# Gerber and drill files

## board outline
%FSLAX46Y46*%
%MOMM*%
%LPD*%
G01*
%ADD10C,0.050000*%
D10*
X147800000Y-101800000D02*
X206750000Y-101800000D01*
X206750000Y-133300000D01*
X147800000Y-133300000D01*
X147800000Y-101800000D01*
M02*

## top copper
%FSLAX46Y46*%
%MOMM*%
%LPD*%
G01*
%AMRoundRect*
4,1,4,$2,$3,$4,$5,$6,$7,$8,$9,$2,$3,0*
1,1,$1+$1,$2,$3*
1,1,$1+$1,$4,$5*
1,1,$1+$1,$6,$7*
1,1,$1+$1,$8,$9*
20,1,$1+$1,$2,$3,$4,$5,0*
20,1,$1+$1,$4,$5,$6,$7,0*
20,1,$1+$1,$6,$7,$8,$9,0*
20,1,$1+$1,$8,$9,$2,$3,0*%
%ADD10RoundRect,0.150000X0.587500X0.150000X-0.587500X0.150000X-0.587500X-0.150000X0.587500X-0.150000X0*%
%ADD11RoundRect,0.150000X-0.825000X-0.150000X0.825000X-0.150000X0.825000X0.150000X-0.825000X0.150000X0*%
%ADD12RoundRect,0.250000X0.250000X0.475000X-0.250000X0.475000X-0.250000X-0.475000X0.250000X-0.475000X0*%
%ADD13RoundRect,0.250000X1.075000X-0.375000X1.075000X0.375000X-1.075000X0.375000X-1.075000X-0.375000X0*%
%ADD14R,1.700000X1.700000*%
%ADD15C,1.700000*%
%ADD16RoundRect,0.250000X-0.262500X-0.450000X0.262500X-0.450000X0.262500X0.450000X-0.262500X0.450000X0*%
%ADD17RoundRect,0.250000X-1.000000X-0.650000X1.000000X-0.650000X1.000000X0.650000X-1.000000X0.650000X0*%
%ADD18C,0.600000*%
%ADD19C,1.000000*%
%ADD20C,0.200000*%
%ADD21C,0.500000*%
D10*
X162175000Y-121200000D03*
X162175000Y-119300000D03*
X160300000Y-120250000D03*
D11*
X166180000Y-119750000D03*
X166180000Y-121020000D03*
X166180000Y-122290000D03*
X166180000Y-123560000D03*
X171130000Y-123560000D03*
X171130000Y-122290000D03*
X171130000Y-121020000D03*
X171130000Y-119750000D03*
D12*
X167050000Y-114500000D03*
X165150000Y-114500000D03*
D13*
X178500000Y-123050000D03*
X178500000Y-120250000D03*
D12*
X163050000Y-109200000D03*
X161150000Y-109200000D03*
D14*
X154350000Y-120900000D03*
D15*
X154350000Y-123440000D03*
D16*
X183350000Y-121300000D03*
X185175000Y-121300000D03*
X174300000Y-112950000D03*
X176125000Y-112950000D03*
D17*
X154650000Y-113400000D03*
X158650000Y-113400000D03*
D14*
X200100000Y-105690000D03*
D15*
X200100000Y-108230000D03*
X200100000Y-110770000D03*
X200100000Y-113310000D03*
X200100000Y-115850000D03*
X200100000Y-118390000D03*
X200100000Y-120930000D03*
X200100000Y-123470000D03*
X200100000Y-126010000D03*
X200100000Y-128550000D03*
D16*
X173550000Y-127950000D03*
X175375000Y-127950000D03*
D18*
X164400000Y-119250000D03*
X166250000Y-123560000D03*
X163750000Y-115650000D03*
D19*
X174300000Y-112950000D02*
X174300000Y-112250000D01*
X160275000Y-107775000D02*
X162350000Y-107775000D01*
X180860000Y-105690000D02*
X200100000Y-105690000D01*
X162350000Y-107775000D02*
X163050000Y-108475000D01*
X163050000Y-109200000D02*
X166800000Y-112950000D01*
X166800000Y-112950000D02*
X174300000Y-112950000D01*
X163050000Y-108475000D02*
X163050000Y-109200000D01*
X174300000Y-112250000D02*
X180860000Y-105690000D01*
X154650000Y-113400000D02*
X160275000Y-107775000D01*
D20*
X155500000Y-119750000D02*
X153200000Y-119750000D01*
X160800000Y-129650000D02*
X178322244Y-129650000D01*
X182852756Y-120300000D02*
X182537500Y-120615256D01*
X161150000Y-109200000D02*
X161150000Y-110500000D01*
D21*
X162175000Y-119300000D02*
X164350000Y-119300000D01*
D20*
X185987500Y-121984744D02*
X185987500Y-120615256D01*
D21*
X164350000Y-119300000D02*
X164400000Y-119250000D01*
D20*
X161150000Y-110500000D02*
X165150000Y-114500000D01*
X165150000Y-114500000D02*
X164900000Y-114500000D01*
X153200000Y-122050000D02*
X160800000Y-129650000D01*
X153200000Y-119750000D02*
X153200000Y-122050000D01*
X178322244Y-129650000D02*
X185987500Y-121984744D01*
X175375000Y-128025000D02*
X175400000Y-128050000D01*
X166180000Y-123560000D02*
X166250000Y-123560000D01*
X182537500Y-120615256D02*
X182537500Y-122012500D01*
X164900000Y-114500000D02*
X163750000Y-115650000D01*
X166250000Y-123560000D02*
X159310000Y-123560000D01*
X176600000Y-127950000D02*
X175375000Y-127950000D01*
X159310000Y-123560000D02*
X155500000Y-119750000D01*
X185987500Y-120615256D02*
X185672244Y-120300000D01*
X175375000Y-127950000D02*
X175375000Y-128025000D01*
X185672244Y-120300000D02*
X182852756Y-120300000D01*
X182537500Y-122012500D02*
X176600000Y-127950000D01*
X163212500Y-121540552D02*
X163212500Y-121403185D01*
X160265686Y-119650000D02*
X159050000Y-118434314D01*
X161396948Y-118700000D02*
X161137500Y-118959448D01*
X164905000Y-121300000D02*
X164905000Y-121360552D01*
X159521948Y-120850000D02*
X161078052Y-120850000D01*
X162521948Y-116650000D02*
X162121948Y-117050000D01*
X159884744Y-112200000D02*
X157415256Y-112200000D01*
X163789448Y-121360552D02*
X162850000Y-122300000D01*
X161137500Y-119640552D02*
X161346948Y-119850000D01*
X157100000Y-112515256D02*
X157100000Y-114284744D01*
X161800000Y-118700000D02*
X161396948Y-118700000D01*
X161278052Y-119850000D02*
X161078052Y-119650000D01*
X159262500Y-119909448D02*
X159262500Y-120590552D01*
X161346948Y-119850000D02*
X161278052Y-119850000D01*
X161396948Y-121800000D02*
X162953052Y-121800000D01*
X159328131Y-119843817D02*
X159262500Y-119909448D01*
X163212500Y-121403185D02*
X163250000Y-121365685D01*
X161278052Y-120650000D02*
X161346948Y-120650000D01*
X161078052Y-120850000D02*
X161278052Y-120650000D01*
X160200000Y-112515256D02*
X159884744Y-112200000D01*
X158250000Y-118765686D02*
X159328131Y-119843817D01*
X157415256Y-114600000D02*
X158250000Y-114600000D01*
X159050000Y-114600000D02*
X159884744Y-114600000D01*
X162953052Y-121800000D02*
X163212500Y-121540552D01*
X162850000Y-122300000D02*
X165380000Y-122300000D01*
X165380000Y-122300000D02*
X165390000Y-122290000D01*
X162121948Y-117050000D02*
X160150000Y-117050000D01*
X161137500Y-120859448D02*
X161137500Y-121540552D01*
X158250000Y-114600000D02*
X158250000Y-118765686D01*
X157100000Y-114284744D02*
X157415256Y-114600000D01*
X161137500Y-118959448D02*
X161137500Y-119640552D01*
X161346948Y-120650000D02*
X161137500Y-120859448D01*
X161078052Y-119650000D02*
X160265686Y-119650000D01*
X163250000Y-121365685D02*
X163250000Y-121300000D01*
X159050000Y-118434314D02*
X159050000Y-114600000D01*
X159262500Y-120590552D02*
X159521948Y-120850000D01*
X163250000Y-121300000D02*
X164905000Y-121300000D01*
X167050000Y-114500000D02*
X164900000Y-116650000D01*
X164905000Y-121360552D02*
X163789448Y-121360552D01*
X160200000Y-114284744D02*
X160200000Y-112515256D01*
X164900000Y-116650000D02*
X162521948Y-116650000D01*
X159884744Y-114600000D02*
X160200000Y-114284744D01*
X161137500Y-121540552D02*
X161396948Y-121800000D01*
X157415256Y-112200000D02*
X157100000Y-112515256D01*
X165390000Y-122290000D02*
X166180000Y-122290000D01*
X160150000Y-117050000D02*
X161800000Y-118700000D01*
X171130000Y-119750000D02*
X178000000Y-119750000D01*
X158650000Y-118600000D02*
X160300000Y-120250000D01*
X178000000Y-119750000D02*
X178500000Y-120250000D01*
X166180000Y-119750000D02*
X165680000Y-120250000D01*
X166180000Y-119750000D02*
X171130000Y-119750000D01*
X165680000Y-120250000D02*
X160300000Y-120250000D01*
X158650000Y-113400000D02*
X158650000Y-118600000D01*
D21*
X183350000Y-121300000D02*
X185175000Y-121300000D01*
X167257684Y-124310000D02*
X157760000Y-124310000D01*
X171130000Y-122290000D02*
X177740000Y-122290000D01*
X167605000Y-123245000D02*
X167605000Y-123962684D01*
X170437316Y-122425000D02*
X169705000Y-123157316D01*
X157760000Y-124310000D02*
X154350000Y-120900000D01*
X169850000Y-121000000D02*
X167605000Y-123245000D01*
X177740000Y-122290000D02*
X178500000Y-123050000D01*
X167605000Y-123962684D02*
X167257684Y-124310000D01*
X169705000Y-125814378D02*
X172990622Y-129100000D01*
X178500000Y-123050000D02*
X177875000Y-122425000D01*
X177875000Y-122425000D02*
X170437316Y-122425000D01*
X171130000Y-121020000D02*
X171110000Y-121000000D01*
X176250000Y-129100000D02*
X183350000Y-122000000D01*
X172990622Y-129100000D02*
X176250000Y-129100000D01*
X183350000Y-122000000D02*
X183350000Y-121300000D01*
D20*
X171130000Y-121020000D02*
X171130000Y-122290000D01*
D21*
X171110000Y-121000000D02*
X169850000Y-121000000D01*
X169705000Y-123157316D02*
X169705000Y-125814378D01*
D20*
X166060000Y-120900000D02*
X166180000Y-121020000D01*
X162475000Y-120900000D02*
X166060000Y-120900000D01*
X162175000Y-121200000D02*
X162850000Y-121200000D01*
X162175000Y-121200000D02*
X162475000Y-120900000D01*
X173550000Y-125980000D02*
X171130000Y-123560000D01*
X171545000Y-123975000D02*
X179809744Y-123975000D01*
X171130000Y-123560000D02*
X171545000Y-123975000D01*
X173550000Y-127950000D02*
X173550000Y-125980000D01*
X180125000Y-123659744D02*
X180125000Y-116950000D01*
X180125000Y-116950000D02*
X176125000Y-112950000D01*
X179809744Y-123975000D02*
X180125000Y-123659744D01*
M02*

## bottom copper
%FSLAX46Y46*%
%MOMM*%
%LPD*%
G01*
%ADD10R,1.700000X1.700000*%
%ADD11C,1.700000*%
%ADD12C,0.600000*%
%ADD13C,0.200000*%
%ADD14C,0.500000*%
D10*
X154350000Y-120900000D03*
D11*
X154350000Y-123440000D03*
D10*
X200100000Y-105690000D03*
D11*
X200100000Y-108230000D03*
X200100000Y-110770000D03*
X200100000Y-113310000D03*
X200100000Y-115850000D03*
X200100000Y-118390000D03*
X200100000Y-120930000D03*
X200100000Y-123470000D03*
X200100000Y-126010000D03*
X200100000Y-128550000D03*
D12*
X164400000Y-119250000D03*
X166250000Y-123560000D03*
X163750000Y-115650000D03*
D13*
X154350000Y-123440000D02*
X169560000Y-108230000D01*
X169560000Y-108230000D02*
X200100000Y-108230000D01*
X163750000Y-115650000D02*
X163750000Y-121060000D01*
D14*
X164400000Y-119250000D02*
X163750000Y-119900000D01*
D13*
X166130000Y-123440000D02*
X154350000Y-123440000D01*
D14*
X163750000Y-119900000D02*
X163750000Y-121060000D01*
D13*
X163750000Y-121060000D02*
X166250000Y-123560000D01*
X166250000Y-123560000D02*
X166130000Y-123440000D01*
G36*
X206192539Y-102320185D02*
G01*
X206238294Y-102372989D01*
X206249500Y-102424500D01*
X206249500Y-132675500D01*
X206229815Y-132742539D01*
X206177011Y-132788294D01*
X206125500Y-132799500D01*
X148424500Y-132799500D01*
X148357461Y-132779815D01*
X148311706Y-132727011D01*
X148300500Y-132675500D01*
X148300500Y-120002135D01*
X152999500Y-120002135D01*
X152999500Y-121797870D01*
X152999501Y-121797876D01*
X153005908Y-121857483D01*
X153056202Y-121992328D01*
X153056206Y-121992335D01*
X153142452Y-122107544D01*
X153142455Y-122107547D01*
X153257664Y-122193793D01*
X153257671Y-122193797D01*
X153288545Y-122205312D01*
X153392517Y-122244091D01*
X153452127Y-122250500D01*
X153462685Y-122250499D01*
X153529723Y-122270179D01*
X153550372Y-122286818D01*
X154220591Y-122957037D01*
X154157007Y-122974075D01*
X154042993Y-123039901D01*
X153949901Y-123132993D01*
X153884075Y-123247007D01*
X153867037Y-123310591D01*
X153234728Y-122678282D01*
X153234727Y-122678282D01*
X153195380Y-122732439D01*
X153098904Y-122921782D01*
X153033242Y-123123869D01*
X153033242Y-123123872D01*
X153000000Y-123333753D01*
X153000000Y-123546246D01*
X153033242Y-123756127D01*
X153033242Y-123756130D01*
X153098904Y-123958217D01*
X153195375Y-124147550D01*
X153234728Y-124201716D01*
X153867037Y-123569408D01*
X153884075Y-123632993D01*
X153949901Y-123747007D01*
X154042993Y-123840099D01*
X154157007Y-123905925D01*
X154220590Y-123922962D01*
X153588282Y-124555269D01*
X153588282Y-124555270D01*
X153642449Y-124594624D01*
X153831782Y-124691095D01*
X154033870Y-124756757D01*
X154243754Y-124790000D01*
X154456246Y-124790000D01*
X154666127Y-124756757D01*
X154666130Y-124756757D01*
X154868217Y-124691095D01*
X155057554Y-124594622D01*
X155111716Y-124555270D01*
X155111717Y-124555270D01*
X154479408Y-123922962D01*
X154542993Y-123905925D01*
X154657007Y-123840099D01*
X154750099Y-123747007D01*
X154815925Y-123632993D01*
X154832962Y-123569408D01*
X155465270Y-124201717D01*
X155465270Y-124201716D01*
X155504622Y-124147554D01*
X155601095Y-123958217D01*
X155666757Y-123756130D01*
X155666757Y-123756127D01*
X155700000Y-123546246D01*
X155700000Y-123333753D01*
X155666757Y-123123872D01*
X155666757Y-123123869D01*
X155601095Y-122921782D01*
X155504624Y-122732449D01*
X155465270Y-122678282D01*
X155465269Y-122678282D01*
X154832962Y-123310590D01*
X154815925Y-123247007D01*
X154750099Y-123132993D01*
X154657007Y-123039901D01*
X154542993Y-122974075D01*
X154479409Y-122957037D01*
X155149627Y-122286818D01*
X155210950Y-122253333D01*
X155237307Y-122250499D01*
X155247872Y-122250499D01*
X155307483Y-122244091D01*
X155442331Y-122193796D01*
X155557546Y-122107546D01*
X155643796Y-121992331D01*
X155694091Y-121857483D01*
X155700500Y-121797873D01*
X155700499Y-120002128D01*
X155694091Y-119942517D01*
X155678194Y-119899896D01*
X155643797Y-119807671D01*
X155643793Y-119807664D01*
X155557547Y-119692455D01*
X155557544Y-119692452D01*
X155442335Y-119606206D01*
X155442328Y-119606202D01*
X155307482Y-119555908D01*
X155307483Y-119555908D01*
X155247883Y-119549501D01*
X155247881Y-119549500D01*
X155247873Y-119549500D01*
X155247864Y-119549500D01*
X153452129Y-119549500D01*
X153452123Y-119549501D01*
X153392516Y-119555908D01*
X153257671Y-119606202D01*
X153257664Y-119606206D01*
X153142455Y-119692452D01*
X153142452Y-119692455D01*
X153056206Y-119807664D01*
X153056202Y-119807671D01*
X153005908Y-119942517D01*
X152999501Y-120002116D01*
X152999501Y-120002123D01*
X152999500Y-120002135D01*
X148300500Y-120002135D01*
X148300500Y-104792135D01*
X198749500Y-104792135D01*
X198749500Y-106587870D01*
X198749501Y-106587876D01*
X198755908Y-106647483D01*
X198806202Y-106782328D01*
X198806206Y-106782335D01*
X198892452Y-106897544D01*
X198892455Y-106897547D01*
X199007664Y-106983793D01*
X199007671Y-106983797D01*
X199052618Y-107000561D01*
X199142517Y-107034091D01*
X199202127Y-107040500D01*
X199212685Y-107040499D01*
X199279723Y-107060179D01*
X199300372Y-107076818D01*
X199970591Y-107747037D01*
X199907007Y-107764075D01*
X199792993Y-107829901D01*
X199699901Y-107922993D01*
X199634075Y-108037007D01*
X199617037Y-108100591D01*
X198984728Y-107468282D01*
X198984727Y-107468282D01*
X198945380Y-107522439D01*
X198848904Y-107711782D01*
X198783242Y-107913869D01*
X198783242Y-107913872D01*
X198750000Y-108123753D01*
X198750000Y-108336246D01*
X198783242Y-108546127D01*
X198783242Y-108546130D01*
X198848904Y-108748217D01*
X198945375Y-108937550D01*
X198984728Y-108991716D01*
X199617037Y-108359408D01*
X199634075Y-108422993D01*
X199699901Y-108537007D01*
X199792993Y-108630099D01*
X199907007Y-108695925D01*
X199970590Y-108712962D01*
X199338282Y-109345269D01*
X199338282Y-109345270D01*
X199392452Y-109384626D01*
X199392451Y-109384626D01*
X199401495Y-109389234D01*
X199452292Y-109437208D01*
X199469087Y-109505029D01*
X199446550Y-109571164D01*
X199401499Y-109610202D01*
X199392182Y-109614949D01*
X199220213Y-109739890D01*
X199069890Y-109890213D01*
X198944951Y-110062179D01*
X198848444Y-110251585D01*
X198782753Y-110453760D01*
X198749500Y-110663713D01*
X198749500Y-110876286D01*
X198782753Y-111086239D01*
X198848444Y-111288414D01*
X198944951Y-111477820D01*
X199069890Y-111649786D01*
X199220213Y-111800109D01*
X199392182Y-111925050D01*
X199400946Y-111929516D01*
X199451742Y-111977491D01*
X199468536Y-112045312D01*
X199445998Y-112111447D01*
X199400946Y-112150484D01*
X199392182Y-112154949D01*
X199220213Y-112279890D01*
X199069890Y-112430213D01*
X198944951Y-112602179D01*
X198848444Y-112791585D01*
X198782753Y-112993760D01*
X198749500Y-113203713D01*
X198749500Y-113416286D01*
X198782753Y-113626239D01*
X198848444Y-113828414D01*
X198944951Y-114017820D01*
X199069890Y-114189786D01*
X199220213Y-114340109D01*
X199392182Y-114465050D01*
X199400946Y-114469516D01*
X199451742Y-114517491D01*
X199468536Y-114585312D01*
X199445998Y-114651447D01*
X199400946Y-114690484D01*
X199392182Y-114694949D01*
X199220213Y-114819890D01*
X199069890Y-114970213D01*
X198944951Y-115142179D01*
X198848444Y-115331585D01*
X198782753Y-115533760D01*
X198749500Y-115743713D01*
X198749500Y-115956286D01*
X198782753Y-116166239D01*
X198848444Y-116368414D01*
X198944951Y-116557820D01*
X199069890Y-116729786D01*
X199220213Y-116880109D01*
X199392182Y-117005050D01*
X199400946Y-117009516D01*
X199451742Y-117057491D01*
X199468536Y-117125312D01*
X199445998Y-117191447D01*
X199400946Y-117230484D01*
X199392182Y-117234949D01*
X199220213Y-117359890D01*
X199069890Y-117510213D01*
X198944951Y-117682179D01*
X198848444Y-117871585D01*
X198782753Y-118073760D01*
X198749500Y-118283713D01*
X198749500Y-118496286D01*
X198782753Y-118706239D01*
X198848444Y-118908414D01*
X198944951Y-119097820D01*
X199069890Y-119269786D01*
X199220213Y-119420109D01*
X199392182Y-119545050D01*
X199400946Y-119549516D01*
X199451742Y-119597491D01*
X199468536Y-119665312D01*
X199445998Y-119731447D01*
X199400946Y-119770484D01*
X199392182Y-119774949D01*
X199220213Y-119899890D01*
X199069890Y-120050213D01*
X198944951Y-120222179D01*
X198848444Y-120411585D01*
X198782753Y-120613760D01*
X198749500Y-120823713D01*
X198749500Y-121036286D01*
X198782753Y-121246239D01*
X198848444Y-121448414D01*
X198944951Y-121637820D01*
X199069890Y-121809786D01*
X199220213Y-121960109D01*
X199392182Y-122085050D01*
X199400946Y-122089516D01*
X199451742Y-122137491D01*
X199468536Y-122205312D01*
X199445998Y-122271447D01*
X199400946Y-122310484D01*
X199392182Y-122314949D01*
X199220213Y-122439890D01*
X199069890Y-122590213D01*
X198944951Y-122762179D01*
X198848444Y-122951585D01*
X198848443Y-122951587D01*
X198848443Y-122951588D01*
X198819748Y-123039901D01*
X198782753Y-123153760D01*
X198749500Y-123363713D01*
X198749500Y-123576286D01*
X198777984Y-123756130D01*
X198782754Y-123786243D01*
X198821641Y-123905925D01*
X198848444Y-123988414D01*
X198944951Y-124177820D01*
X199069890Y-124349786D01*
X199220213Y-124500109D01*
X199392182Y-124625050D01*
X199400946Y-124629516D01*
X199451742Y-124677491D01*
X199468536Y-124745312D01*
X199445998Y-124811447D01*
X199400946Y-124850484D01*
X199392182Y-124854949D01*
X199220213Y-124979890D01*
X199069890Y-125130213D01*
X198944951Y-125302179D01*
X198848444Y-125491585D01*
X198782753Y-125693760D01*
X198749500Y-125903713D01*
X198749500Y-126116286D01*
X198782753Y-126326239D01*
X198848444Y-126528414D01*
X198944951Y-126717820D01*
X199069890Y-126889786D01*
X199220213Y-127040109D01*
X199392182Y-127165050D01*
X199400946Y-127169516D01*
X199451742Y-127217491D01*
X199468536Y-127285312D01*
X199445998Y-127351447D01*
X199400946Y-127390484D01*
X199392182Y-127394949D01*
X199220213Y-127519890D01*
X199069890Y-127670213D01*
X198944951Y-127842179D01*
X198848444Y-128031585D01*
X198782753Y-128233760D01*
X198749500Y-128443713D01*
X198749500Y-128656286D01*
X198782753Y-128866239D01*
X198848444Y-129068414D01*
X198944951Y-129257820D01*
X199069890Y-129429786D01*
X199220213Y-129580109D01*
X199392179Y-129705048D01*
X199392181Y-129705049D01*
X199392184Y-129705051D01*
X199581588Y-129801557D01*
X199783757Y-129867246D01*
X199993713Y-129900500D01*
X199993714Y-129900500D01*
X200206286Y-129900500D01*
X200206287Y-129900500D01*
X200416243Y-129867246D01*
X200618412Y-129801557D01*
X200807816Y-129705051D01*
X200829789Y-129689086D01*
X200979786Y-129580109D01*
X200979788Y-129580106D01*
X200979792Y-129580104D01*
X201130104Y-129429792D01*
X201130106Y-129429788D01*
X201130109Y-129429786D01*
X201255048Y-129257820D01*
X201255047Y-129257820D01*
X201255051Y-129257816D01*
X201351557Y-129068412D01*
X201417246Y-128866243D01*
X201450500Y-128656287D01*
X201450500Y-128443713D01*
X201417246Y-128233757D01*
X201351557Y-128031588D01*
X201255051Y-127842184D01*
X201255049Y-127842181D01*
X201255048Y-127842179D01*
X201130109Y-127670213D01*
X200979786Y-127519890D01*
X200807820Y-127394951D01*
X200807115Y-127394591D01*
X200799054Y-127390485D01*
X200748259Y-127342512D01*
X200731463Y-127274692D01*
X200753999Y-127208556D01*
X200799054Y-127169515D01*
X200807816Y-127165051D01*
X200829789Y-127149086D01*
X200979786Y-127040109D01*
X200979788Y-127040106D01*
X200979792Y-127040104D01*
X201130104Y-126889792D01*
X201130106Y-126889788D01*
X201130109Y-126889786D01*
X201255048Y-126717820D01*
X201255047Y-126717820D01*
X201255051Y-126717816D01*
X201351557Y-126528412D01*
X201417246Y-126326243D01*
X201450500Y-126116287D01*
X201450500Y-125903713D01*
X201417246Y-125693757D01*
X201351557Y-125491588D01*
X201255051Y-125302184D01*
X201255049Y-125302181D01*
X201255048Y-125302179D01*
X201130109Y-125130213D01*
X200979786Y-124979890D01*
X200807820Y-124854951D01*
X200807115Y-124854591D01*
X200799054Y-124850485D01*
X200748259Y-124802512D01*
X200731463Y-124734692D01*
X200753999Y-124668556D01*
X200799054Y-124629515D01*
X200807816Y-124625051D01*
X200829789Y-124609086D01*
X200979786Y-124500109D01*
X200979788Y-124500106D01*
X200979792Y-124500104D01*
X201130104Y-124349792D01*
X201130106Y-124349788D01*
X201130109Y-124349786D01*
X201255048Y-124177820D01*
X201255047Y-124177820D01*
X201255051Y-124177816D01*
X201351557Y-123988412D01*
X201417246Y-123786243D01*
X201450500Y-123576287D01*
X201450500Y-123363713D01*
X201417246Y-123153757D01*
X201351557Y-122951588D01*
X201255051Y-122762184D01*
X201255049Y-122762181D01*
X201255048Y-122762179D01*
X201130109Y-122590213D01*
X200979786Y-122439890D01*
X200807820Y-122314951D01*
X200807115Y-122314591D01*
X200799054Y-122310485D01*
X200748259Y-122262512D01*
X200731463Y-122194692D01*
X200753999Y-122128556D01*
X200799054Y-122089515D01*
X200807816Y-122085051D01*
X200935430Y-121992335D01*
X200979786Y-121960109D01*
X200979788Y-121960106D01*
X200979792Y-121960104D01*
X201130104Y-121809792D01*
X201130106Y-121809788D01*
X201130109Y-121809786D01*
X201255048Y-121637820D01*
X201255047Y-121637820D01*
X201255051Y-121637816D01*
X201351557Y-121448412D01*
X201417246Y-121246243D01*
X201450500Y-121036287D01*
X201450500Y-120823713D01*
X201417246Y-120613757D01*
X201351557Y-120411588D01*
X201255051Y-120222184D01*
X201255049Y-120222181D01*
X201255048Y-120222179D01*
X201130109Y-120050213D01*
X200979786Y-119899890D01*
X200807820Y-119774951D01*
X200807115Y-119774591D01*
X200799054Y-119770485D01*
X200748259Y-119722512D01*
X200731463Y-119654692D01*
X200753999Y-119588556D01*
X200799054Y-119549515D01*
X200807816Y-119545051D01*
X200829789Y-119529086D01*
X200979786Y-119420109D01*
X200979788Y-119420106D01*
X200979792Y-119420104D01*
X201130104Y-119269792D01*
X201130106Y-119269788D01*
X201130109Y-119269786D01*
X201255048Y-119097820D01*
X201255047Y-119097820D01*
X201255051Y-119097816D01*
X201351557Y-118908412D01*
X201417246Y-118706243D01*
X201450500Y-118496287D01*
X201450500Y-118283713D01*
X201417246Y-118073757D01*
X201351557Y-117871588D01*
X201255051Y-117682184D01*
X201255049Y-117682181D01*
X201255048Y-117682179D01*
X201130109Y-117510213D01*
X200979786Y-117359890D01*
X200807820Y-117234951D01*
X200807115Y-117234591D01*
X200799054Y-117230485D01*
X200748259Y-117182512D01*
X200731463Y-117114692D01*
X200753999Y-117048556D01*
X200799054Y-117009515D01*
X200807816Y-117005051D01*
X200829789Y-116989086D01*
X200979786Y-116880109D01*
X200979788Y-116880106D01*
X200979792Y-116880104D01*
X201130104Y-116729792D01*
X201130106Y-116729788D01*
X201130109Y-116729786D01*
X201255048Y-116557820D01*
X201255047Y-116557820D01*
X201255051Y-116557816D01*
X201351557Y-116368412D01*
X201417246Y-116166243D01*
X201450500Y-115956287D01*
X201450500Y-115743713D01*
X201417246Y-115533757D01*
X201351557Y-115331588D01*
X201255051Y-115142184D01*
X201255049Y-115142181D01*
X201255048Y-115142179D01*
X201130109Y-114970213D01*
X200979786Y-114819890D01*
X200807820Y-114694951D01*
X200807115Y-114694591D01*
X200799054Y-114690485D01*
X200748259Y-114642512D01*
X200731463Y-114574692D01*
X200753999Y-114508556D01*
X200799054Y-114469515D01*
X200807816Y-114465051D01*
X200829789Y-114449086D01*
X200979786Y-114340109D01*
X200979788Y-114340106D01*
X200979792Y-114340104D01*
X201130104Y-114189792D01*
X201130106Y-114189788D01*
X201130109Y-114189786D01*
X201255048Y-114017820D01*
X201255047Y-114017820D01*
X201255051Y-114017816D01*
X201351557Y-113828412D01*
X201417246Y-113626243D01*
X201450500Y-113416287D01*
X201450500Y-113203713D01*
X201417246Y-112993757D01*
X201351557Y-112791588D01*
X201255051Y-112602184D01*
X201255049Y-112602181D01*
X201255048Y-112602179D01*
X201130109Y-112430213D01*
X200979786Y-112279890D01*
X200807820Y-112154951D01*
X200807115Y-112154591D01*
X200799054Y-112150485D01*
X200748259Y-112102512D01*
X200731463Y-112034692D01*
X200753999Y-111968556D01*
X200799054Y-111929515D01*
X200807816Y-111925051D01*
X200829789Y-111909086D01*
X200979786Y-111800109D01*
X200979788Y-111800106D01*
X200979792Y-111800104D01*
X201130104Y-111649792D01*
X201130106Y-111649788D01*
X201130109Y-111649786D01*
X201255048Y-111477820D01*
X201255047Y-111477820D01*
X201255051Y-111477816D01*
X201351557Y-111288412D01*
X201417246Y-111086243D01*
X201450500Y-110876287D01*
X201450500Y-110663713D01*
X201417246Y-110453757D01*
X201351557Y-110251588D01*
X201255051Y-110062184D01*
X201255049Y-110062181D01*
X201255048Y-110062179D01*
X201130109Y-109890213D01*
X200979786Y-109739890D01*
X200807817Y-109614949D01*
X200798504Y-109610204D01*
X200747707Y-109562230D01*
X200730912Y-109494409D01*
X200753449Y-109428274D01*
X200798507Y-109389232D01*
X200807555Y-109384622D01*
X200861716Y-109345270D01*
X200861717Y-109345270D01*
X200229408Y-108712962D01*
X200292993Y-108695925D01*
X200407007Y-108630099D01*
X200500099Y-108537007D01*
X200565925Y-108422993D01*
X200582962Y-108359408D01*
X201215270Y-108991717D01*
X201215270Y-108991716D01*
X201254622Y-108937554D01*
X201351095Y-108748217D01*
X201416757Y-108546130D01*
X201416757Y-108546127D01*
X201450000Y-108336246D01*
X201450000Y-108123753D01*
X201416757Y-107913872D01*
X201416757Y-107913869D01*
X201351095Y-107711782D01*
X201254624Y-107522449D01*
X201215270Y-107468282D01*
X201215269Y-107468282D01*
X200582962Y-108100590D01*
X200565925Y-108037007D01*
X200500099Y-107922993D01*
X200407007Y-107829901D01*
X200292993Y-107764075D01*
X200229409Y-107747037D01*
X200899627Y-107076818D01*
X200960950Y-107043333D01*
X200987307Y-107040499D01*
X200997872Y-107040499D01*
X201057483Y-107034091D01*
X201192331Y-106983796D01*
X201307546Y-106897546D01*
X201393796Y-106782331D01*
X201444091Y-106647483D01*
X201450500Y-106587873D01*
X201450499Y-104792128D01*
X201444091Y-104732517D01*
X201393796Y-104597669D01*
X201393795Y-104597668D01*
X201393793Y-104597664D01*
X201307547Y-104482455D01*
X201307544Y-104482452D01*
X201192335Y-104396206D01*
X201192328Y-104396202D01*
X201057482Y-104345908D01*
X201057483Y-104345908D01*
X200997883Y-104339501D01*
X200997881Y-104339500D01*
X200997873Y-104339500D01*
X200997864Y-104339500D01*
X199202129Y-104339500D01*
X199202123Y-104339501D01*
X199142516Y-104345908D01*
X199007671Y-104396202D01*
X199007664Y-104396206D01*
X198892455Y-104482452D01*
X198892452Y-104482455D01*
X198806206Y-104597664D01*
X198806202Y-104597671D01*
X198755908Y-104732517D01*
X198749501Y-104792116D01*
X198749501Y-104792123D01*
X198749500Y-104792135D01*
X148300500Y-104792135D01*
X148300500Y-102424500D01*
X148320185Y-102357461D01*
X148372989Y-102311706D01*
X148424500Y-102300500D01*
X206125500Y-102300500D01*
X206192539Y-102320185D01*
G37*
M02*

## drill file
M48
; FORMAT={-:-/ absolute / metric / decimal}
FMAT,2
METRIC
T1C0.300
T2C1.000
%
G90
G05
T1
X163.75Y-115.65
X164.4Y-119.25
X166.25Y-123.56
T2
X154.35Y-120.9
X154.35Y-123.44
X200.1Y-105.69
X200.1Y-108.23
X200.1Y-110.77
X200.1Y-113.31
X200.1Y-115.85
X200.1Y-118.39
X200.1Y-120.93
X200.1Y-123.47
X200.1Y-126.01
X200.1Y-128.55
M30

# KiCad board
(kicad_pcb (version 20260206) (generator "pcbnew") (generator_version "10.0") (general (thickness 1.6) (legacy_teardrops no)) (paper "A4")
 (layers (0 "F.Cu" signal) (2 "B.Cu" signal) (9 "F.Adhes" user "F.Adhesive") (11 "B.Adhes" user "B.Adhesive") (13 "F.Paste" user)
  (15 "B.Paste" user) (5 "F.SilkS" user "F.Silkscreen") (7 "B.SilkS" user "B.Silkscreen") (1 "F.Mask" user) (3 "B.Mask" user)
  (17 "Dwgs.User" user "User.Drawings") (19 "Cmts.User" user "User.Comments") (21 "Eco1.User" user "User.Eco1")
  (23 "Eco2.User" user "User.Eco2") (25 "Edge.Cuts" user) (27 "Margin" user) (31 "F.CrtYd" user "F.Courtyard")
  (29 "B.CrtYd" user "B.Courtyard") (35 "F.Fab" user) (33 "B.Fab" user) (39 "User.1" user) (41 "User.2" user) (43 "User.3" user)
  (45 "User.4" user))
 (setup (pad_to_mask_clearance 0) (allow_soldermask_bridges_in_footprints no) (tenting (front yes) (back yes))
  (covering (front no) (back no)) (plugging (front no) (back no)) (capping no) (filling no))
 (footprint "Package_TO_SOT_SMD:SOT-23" (layer "F.Cu") (at 161.2375 120.25 180)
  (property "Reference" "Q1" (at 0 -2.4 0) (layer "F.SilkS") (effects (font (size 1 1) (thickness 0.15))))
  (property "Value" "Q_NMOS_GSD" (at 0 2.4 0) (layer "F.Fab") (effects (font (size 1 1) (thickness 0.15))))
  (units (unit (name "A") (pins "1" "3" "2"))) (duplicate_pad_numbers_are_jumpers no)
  (pad "1" smd roundrect (at -0.9375 -0.95 180) (size 1.475 0.6) (layers "F.Cu" "F.Mask" "F.Paste") (roundrect_rratio 0.25)
   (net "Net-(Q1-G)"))
  (pad "2" smd roundrect (at -0.9375 0.95 180) (size 1.475 0.6) (layers "F.Cu" "F.Mask" "F.Paste") (roundrect_rratio 0.25) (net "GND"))
  (pad "3" smd roundrect (at 0.9375 0 180) (size 1.475 0.6) (layers "F.Cu" "F.Mask" "F.Paste") (roundrect_rratio 0.25) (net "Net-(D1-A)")))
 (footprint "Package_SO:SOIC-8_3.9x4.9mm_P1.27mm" (layer "F.Cu") (at 168.655 121.655)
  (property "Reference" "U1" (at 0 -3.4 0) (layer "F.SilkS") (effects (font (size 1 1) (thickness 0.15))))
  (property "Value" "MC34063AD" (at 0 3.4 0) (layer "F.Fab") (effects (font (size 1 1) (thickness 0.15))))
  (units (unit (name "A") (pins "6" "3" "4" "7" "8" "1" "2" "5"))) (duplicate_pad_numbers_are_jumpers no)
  (pad "1" smd roundrect (at -2.475 -1.905) (size 1.95 0.6) (layers "F.Cu" "F.Mask" "F.Paste") (roundrect_rratio 0.25) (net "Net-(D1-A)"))
  (pad "2" smd roundrect (at -2.475 -0.635) (size 1.95 0.6) (layers "F.Cu" "F.Mask" "F.Paste") (roundrect_rratio 0.25) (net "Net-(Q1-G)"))
  (pad "3" smd roundrect (at -2.475 0.635) (size 1.95 0.6) (layers "F.Cu" "F.Mask" "F.Paste") (roundrect_rratio 0.25) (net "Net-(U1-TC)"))
  (pad "4" smd roundrect (at -2.475 1.905) (size 1.95 0.6) (layers "F.Cu" "F.Mask" "F.Paste") (roundrect_rratio 0.25) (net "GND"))
  (pad "5" smd roundrect (at 2.475 1.905) (size 1.95 0.6) (layers "F.Cu" "F.Mask" "F.Paste") (roundrect_rratio 0.25) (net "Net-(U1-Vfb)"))
  (pad "6" smd roundrect (at 2.475 0.635) (size 1.95 0.6) (layers "F.Cu" "F.Mask" "F.Paste") (roundrect_rratio 0.25) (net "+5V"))
  (pad "7" smd roundrect (at 2.475 -0.635) (size 1.95 0.6) (layers "F.Cu" "F.Mask" "F.Paste") (roundrect_rratio 0.25) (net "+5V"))
  (pad "8" smd roundrect (at 2.475 -1.905) (size 1.95 0.6) (layers "F.Cu" "F.Mask" "F.Paste") (roundrect_rratio 0.25) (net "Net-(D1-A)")))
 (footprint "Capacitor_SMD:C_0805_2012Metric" (layer "F.Cu") (at 166.1 114.5 180)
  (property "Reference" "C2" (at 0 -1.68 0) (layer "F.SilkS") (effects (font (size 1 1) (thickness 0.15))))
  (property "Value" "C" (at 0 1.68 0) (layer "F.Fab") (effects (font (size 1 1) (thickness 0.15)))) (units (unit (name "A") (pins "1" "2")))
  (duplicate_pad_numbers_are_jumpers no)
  (pad "1" smd roundrect (at -0.95 0 180) (size 1 1.45) (layers "F.Cu" "F.Mask" "F.Paste") (roundrect_rratio 0.25) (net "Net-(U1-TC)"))
  (pad "2" smd roundrect (at 0.95 0 180) (size 1 1.45) (layers "F.Cu" "F.Mask" "F.Paste") (roundrect_rratio 0.25) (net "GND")))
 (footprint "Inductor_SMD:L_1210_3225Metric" (layer "F.Cu") (at 178.5 121.65 90)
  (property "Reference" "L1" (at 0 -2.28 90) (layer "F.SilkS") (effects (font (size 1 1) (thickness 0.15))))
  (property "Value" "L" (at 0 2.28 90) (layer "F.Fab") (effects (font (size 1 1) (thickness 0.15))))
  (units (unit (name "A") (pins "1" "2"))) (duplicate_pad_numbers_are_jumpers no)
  (pad "1" smd roundrect (at -1.4 0 90) (size 1.25 2.65) (layers "F.Cu" "F.Mask" "F.Paste") (roundrect_rratio 0.2) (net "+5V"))
  (pad "2" smd roundrect (at 1.4 0 90) (size 1.25 2.65) (layers "F.Cu" "F.Mask" "F.Paste") (roundrect_rratio 0.2) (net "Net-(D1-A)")))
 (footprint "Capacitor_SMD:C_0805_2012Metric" (layer "F.Cu") (at 162.1 109.2 180)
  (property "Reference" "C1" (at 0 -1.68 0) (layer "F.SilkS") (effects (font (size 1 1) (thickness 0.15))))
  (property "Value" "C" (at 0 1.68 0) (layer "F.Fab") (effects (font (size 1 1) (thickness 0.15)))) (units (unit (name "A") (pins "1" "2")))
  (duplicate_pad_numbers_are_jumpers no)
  (pad "1" smd roundrect (at -0.95 0 180) (size 1 1.45) (layers "F.Cu" "F.Mask" "F.Paste") (roundrect_rratio 0.25) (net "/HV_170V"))
  (pad "2" smd roundrect (at 0.95 0 180) (size 1 1.45) (layers "F.Cu" "F.Mask" "F.Paste") (roundrect_rratio 0.25) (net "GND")))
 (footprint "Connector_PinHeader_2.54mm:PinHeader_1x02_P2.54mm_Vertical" (layer "F.Cu") (at 154.35 120.9)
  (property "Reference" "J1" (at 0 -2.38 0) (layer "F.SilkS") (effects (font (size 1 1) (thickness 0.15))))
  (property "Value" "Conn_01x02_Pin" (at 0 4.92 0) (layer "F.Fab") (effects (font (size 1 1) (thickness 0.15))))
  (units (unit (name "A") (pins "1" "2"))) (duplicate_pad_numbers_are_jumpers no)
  (pad "1" thru_hole rect (at 0 0) (size 1.7 1.7) (drill 1) (layers "*.Cu" "*.Mask") (remove_unused_layers no) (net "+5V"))
  (pad "2" thru_hole circle (at 0 2.54) (size 1.7 1.7) (drill 1) (layers "*.Cu" "*.Mask") (remove_unused_layers no) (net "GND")))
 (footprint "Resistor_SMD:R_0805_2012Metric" (layer "F.Cu") (at 184.2625 121.3)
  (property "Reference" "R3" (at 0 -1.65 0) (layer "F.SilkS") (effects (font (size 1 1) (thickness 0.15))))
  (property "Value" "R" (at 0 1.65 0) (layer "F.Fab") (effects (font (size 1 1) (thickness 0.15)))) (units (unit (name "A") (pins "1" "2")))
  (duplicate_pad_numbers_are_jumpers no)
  (pad "1" smd roundrect (at -0.9125 0) (size 1.025 1.4) (layers "F.Cu" "F.Mask" "F.Paste") (roundrect_rratio 0.243902) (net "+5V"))
  (pad "2" smd roundrect (at 0.9125 0) (size 1.025 1.4) (layers "F.Cu" "F.Mask" "F.Paste") (roundrect_rratio 0.243902) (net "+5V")))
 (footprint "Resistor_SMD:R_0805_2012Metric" (layer "F.Cu") (at 175.2125 112.95)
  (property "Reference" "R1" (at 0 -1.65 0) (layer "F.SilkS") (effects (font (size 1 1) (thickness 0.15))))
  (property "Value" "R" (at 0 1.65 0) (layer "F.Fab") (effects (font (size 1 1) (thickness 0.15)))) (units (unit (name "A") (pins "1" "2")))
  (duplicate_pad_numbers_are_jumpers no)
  (pad "1" smd roundrect (at -0.9125 0) (size 1.025 1.4) (layers "F.Cu" "F.Mask" "F.Paste") (roundrect_rratio 0.243902) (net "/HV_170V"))
  (pad "2" smd roundrect (at 0.9125 0) (size 1.025 1.4) (layers "F.Cu" "F.Mask" "F.Paste") (roundrect_rratio 0.243902) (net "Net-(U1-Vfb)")))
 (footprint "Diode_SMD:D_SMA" (layer "F.Cu") (at 156.65 113.4)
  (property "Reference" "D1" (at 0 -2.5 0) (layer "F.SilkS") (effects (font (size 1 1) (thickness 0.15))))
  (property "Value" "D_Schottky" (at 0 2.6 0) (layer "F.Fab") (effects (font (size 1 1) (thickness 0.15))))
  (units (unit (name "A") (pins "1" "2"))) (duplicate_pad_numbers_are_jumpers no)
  (pad "1" smd roundrect (at -2 0) (size 2.5 1.8) (layers "F.Cu" "F.Mask" "F.Paste") (roundrect_rratio 0.1388888889) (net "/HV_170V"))
  (pad "2" smd roundrect (at 2 0) (size 2.5 1.8) (layers "F.Cu" "F.Mask" "F.Paste") (roundrect_rratio 0.1388888889) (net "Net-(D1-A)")))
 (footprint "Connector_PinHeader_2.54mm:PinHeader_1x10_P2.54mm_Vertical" (layer "F.Cu") (at 200.1 105.69)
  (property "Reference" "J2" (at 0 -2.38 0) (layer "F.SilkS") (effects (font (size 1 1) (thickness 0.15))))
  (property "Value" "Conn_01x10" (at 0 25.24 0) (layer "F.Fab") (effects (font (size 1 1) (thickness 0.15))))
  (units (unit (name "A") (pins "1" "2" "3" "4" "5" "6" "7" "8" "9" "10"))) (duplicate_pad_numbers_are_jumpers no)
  (pad "1" thru_hole rect (at 0 0) (size 1.7 1.7) (drill 1) (layers "*.Cu" "*.Mask") (remove_unused_layers no) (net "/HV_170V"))
  (pad "2" thru_hole circle (at 0 2.54) (size 1.7 1.7) (drill 1) (layers "*.Cu" "*.Mask") (remove_unused_layers no) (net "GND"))
  (pad "3" thru_hole circle (at 0 5.08) (size 1.7 1.7) (drill 1) (layers "*.Cu" "*.Mask") (remove_unused_layers no) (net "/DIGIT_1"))
  (pad "4" thru_hole circle (at 0 7.62) (size 1.7 1.7) (drill 1) (layers "*.Cu" "*.Mask") (remove_unused_layers no) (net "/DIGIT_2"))
  (pad "5" thru_hole circle (at 0 10.16) (size 1.7 1.7) (drill 1) (layers "*.Cu" "*.Mask") (remove_unused_layers no) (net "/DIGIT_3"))
  (pad "6" thru_hole circle (at 0 12.7) (size 1.7 1.7) (drill 1) (layers "*.Cu" "*.Mask") (remove_unused_layers no) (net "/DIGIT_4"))
  (pad "7" thru_hole circle (at 0 15.24) (size 1.7 1.7) (drill 1) (layers "*.Cu" "*.Mask") (remove_unused_layers no) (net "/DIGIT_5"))
  (pad "8" thru_hole circle (at 0 17.78) (size 1.7 1.7) (drill 1) (layers "*.Cu" "*.Mask") (remove_unused_layers no) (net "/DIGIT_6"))
  (pad "9" thru_hole circle (at 0 20.32) (size 1.7 1.7) (drill 1) (layers "*.Cu" "*.Mask") (remove_unused_layers no) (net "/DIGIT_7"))
  (pad "10" thru_hole circle (at 0 22.86) (size 1.7 1.7) (drill 1) (layers "*.Cu" "*.Mask") (remove_unused_layers no) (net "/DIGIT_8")))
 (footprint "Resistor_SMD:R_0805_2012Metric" (layer "F.Cu") (at 174.4625 127.95)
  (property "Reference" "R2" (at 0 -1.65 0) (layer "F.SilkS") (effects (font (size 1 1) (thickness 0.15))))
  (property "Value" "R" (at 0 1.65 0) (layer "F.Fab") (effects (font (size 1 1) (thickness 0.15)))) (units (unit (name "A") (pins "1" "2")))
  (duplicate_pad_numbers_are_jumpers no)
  (pad "1" smd roundrect (at -0.9125 0) (size 1.025 1.4) (layers "F.Cu" "F.Mask" "F.Paste") (roundrect_rratio 0.243902) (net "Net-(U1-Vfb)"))
  (pad "2" smd roundrect (at 0.9125 0) (size 1.025 1.4) (layers "F.Cu" "F.Mask" "F.Paste") (roundrect_rratio 0.243902) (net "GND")))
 (gr_rect (start 147.8 101.8) (end 206.75 133.3) (stroke (width 0.05) (type default)) (fill no) (layer "Edge.Cuts"))
 (segment (start 174.3 112.95) (end 174.3 112.25) (width 1) (layer "F.Cu") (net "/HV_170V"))
 (segment (start 160.275 107.775) (end 162.35 107.775) (width 1) (layer "F.Cu") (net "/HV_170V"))
 (segment (start 180.86 105.69) (end 200.1 105.69) (width 1) (layer "F.Cu") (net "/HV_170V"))
 (segment (start 162.35 107.775) (end 163.05 108.475) (width 1) (layer "F.Cu") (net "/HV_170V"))
 (segment (start 163.05 109.2) (end 166.8 112.95) (width 1) (layer "F.Cu") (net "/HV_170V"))
 (segment (start 166.8 112.95) (end 174.3 112.95) (width 1) (layer "F.Cu") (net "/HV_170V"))
 (segment (start 163.05 108.475) (end 163.05 109.2) (width 1) (layer "F.Cu") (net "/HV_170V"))
 (segment (start 174.3 112.25) (end 180.86 105.69) (width 1) (layer "F.Cu") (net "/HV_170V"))
 (segment (start 154.65 113.4) (end 160.275 107.775) (width 1) (layer "F.Cu") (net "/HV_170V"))
 (segment (start 155.5 119.75) (end 153.2 119.75) (width 0.2) (layer "F.Cu") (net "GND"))
 (segment (start 160.8 129.65) (end 178.322244 129.65) (width 0.2) (layer "F.Cu") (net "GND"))
 (segment (start 182.852756 120.3) (end 182.5375 120.615256) (width 0.2) (layer "F.Cu") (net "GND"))
 (segment (start 161.15 109.2) (end 161.15 110.5) (width 0.2) (layer "F.Cu") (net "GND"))
 (segment (start 162.175 119.3) (end 164.35 119.3) (width 0.5) (layer "F.Cu") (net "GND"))
 (segment (start 185.9875 121.984744) (end 185.9875 120.615256) (width 0.2) (layer "F.Cu") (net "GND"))
 (segment (start 164.35 119.3) (end 164.4 119.25) (width 0.5) (layer "F.Cu") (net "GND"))
 (segment (start 161.15 110.5) (end 165.15 114.5) (width 0.2) (layer "F.Cu") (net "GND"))
 (segment (start 165.15 114.5) (end 164.9 114.5) (width 0.2) (layer "F.Cu") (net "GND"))
 (segment (start 153.2 122.05) (end 160.8 129.65) (width 0.2) (layer "F.Cu") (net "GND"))
 (segment (start 153.2 119.75) (end 153.2 122.05) (width 0.2) (layer "F.Cu") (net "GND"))
 (segment (start 178.322244 129.65) (end 185.9875 121.984744) (width 0.2) (layer "F.Cu") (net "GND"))
 (segment (start 175.375 128.025) (end 175.4 128.05) (width 0.2) (layer "F.Cu") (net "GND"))
 (segment (start 166.18 123.56) (end 166.25 123.56) (width 0.2) (layer "F.Cu") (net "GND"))
 (segment (start 182.5375 120.615256) (end 182.5375 122.0125) (width 0.2) (layer "F.Cu") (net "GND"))
 (segment (start 164.9 114.5) (end 163.75 115.65) (width 0.2) (layer "F.Cu") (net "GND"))
 (segment (start 166.25 123.56) (end 159.31 123.56) (width 0.2) (layer "F.Cu") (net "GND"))
 (segment (start 176.6 127.95) (end 175.375 127.95) (width 0.2) (layer "F.Cu") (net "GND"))
 (segment (start 159.31 123.56) (end 155.5 119.75) (width 0.2) (layer "F.Cu") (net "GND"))
 (segment (start 185.9875 120.615256) (end 185.672244 120.3) (width 0.2) (layer "F.Cu") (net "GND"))
 (segment (start 175.375 127.95) (end 175.375 128.025) (width 0.2) (layer "F.Cu") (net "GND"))
 (segment (start 185.672244 120.3) (end 182.852756 120.3) (width 0.2) (layer "F.Cu") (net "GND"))
 (segment (start 182.5375 122.0125) (end 176.6 127.95) (width 0.2) (layer "F.Cu") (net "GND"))
 (via (at 164.4 119.25) (size 0.6) (drill 0.3) (layers "F.Cu" "B.Cu") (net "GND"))
 (via (at 166.25 123.56) (size 0.6) (drill 0.3) (layers "F.Cu" "B.Cu") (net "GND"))
 (via (at 163.75 115.65) (size 0.6) (drill 0.3) (layers "F.Cu" "B.Cu") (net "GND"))
 (segment (start 154.35 123.44) (end 169.56 108.23) (width 0.2) (layer "B.Cu") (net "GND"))
 (segment (start 169.56 108.23) (end 200.1 108.23) (width 0.2) (layer "B.Cu") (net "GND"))
 (segment (start 163.75 115.65) (end 163.75 121.06) (width 0.2) (layer "B.Cu") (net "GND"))
 (segment (start 164.4 119.25) (end 163.75 119.9) (width 0.5) (layer "B.Cu") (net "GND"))
 (segment (start 166.13 123.44) (end 154.35 123.44) (width 0.2) (layer "B.Cu") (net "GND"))
 (segment (start 163.75 119.9) (end 163.75 121.06) (width 0.5) (layer "B.Cu") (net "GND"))
 (segment (start 163.75 121.06) (end 166.25 123.56) (width 0.2) (layer "B.Cu") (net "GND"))
 (segment (start 166.25 123.56) (end 166.13 123.44) (width 0.2) (layer "B.Cu") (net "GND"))
 (segment (start 163.2125 121.540552) (end 163.2125 121.403185) (width 0.2) (layer "F.Cu") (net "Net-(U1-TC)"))
 (segment (start 160.265686 119.65) (end 159.05 118.434314) (width 0.2) (layer "F.Cu") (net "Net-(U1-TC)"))
 (segment (start 161.396948 118.7) (end 161.1375 118.959448) (width 0.2) (layer "F.Cu") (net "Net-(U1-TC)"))
 (segment (start 164.905 121.3) (end 164.905 121.360552) (width 0.2) (layer "F.Cu") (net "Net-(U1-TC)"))
 (segment (start 159.521948 120.85) (end 161.078052 120.85) (width 0.2) (layer "F.Cu") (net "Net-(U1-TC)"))
 (segment (start 162.521948 116.65) (end 162.121948 117.05) (width 0.2) (layer "F.Cu") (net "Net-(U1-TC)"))
 (segment (start 159.884744 112.2) (end 157.415256 112.2) (width 0.2) (layer "F.Cu") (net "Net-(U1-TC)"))
 (segment (start 163.789448 121.360552) (end 162.85 122.3) (width 0.2) (layer "F.Cu") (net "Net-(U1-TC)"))
 (segment (start 161.1375 119.640552) (end 161.346948 119.85) (width 0.2) (layer "F.Cu") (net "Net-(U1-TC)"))
 (segment (start 157.1 112.515256) (end 157.1 114.284744) (width 0.2) (layer "F.Cu") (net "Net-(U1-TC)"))
 (segment (start 161.8 118.7) (end 161.396948 118.7) (width 0.2) (layer "F.Cu") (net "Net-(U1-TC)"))
 (segment (start 161.278052 119.85) (end 161.078052 119.65) (width 0.2) (layer "F.Cu") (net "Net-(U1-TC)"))
 (segment (start 159.2625 119.909448) (end 159.2625 120.590552) (width 0.2) (layer "F.Cu") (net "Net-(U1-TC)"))
 (segment (start 161.346948 119.85) (end 161.278052 119.85) (width 0.2) (layer "F.Cu") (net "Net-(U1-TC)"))
 (segment (start 161.396948 121.8) (end 162.953052 121.8) (width 0.2) (layer "F.Cu") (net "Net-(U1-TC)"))
 (segment (start 159.328131 119.843817) (end 159.2625 119.909448) (width 0.2) (layer "F.Cu") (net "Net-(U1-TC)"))
 (segment (start 163.2125 121.403185) (end 163.25 121.365685) (width 0.2) (layer "F.Cu") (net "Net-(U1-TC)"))
 (segment (start 161.278052 120.65) (end 161.346948 120.65) (width 0.2) (layer "F.Cu") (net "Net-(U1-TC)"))
 (segment (start 161.078052 120.85) (end 161.278052 120.65) (width 0.2) (layer "F.Cu") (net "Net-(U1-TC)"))
 (segment (start 160.2 112.515256) (end 159.884744 112.2) (width 0.2) (layer "F.Cu") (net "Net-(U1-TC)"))
 (segment (start 158.25 118.765686) (end 159.328131 119.843817) (width 0.2) (layer "F.Cu") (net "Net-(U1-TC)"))
 (segment (start 157.415256 114.6) (end 158.25 114.6) (width 0.2) (layer "F.Cu") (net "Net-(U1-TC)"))
 (segment (start 159.05 114.6) (end 159.884744 114.6) (width 0.2) (layer "F.Cu") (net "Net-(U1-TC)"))
 (segment (start 162.953052 121.8) (end 163.2125 121.540552) (width 0.2) (layer "F.Cu") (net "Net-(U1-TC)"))
 (segment (start 162.85 122.3) (end 165.38 122.3) (width 0.2) (layer "F.Cu") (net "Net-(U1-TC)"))
 (segment (start 165.38 122.3) (end 165.39 122.29) (width 0.2) (layer "F.Cu") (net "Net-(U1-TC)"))
 (segment (start 162.121948 117.05) (end 160.15 117.05) (width 0.2) (layer "F.Cu") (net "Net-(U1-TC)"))
 (segment (start 161.1375 120.859448) (end 161.1375 121.540552) (width 0.2) (layer "F.Cu") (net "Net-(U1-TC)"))
 (segment (start 158.25 114.6) (end 158.25 118.765686) (width 0.2) (layer "F.Cu") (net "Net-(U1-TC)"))
 (segment (start 157.1 114.284744) (end 157.415256 114.6) (width 0.2) (layer "F.Cu") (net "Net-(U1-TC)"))
 (segment (start 161.1375 118.959448) (end 161.1375 119.640552) (width 0.2) (layer "F.Cu") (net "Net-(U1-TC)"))
 (segment (start 161.346948 120.65) (end 161.1375 120.859448) (width 0.2) (layer "F.Cu") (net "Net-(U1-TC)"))
 (segment (start 161.078052 119.65) (end 160.265686 119.65) (width 0.2) (layer "F.Cu") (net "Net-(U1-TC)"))
 (segment (start 163.25 121.365685) (end 163.25 121.3) (width 0.2) (layer "F.Cu") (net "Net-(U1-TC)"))
 (segment (start 159.05 118.434314) (end 159.05 114.6) (width 0.2) (layer "F.Cu") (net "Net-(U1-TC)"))
 (segment (start 159.2625 120.590552) (end 159.521948 120.85) (width 0.2) (layer "F.Cu") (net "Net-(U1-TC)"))
 (segment (start 163.25 121.3) (end 164.905 121.3) (width 0.2) (layer "F.Cu") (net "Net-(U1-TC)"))
 (segment (start 167.05 114.5) (end 164.9 116.65) (width 0.2) (layer "F.Cu") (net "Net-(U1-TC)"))
 (segment (start 164.905 121.360552) (end 163.789448 121.360552) (width 0.2) (layer "F.Cu") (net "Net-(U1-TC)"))
 (segment (start 160.2 114.284744) (end 160.2 112.515256) (width 0.2) (layer "F.Cu") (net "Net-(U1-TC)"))
 (segment (start 164.9 116.65) (end 162.521948 116.65) (width 0.2) (layer "F.Cu") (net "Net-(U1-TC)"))
 (segment (start 159.884744 114.6) (end 160.2 114.284744) (width 0.2) (layer "F.Cu") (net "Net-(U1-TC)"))
 (segment (start 161.1375 121.540552) (end 161.396948 121.8) (width 0.2) (layer "F.Cu") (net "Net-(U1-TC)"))
 (segment (start 157.415256 112.2) (end 157.1 112.515256) (width 0.2) (layer "F.Cu") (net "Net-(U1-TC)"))
 (segment (start 165.39 122.29) (end 166.18 122.29) (width 0.2) (layer "F.Cu") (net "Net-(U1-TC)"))
 (segment (start 160.15 117.05) (end 161.8 118.7) (width 0.2) (layer "F.Cu") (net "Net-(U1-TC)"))
 (segment (start 171.13 119.75) (end 178 119.75) (width 0.2) (layer "F.Cu") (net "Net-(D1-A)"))
 (segment (start 158.65 118.6) (end 160.3 120.25) (width 0.2) (layer "F.Cu") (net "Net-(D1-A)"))
 (segment (start 178 119.75) (end 178.5 120.25) (width 0.2) (layer "F.Cu") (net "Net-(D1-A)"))
 (segment (start 166.18 119.75) (end 165.68 120.25) (width 0.2) (layer "F.Cu") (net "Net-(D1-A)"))
 (segment (start 166.18 119.75) (end 171.13 119.75) (width 0.2) (layer "F.Cu") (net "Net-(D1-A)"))
 (segment (start 165.68 120.25) (end 160.3 120.25) (width 0.2) (layer "F.Cu") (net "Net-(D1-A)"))
 (segment (start 158.65 113.4) (end 158.65 118.6) (width 0.2) (layer "F.Cu") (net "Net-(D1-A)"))
 (segment (start 183.35 121.3) (end 185.175 121.3) (width 0.5) (layer "F.Cu") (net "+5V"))
 (segment (start 167.257684 124.31) (end 157.76 124.31) (width 0.5) (layer "F.Cu") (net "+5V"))
 (segment (start 171.13 122.29) (end 177.74 122.29) (width 0.5) (layer "F.Cu") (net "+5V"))
 (segment (start 167.605 123.245) (end 167.605 123.962684) (width 0.5) (layer "F.Cu") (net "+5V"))
 (segment (start 170.437316 122.425) (end 169.705 123.157316) (width 0.5) (layer "F.Cu") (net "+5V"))
 (segment (start 157.76 124.31) (end 154.35 120.9) (width 0.5) (layer "F.Cu") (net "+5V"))
 (segment (start 169.85 121) (end 167.605 123.245) (width 0.5) (layer "F.Cu") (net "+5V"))
 (segment (start 177.74 122.29) (end 178.5 123.05) (width 0.5) (layer "F.Cu") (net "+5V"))
 (segment (start 167.605 123.962684) (end 167.257684 124.31) (width 0.5) (layer "F.Cu") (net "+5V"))
 (segment (start 169.705 125.814378) (end 172.990622 129.1) (width 0.5) (layer "F.Cu") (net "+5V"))
 (segment (start 178.5 123.05) (end 177.875 122.425) (width 0.5) (layer "F.Cu") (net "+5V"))
 (segment (start 177.875 122.425) (end 170.437316 122.425) (width 0.5) (layer "F.Cu") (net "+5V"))
 (segment (start 171.13 121.02) (end 171.11 121) (width 0.5) (layer "F.Cu") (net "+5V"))
 (segment (start 176.25 129.1) (end 183.35 122) (width 0.5) (layer "F.Cu") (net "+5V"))
 (segment (start 172.990622 129.1) (end 176.25 129.1) (width 0.5) (layer "F.Cu") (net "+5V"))
 (segment (start 183.35 122) (end 183.35 121.3) (width 0.5) (layer "F.Cu") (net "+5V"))
 (segment (start 171.13 121.02) (end 171.13 122.29) (width 0.2) (layer "F.Cu") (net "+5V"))
 (segment (start 171.11 121) (end 169.85 121) (width 0.5) (layer "F.Cu") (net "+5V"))
 (segment (start 169.705 123.157316) (end 169.705 125.814378) (width 0.5) (layer "F.Cu") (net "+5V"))
 (segment (start 166.06 120.9) (end 166.18 121.02) (width 0.2) (layer "F.Cu") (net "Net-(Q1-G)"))
 (segment (start 162.475 120.9) (end 166.06 120.9) (width 0.2) (layer "F.Cu") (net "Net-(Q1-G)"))
 (segment (start 162.175 121.2) (end 162.85 121.2) (width 0.2) (layer "F.Cu") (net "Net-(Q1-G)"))
 (segment (start 162.175 121.2) (end 162.475 120.9) (width 0.2) (layer "F.Cu") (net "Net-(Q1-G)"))
 (segment (start 173.55 125.98) (end 171.13 123.56) (width 0.2) (layer "F.Cu") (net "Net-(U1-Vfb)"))
 (segment (start 171.545 123.975) (end 179.809744 123.975) (width 0.2) (layer "F.Cu") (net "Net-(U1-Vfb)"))
 (segment (start 171.13 123.56) (end 171.545 123.975) (width 0.2) (layer "F.Cu") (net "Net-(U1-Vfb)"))
 (segment (start 173.55 127.95) (end 173.55 125.98) (width 0.2) (layer "F.Cu") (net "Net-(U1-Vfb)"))
 (segment (start 180.125 123.659744) (end 180.125 116.95) (width 0.2) (layer "F.Cu") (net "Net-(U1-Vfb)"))
 (segment (start 180.125 116.95) (end 176.125 112.95) (width 0.2) (layer "F.Cu") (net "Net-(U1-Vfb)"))
 (segment (start 179.809744 123.975) (end 180.125 123.659744) (width 0.2) (layer "F.Cu") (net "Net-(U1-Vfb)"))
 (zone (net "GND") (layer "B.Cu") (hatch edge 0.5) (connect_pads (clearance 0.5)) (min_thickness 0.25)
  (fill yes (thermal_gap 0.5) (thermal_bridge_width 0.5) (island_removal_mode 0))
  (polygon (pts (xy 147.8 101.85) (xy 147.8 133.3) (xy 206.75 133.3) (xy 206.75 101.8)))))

